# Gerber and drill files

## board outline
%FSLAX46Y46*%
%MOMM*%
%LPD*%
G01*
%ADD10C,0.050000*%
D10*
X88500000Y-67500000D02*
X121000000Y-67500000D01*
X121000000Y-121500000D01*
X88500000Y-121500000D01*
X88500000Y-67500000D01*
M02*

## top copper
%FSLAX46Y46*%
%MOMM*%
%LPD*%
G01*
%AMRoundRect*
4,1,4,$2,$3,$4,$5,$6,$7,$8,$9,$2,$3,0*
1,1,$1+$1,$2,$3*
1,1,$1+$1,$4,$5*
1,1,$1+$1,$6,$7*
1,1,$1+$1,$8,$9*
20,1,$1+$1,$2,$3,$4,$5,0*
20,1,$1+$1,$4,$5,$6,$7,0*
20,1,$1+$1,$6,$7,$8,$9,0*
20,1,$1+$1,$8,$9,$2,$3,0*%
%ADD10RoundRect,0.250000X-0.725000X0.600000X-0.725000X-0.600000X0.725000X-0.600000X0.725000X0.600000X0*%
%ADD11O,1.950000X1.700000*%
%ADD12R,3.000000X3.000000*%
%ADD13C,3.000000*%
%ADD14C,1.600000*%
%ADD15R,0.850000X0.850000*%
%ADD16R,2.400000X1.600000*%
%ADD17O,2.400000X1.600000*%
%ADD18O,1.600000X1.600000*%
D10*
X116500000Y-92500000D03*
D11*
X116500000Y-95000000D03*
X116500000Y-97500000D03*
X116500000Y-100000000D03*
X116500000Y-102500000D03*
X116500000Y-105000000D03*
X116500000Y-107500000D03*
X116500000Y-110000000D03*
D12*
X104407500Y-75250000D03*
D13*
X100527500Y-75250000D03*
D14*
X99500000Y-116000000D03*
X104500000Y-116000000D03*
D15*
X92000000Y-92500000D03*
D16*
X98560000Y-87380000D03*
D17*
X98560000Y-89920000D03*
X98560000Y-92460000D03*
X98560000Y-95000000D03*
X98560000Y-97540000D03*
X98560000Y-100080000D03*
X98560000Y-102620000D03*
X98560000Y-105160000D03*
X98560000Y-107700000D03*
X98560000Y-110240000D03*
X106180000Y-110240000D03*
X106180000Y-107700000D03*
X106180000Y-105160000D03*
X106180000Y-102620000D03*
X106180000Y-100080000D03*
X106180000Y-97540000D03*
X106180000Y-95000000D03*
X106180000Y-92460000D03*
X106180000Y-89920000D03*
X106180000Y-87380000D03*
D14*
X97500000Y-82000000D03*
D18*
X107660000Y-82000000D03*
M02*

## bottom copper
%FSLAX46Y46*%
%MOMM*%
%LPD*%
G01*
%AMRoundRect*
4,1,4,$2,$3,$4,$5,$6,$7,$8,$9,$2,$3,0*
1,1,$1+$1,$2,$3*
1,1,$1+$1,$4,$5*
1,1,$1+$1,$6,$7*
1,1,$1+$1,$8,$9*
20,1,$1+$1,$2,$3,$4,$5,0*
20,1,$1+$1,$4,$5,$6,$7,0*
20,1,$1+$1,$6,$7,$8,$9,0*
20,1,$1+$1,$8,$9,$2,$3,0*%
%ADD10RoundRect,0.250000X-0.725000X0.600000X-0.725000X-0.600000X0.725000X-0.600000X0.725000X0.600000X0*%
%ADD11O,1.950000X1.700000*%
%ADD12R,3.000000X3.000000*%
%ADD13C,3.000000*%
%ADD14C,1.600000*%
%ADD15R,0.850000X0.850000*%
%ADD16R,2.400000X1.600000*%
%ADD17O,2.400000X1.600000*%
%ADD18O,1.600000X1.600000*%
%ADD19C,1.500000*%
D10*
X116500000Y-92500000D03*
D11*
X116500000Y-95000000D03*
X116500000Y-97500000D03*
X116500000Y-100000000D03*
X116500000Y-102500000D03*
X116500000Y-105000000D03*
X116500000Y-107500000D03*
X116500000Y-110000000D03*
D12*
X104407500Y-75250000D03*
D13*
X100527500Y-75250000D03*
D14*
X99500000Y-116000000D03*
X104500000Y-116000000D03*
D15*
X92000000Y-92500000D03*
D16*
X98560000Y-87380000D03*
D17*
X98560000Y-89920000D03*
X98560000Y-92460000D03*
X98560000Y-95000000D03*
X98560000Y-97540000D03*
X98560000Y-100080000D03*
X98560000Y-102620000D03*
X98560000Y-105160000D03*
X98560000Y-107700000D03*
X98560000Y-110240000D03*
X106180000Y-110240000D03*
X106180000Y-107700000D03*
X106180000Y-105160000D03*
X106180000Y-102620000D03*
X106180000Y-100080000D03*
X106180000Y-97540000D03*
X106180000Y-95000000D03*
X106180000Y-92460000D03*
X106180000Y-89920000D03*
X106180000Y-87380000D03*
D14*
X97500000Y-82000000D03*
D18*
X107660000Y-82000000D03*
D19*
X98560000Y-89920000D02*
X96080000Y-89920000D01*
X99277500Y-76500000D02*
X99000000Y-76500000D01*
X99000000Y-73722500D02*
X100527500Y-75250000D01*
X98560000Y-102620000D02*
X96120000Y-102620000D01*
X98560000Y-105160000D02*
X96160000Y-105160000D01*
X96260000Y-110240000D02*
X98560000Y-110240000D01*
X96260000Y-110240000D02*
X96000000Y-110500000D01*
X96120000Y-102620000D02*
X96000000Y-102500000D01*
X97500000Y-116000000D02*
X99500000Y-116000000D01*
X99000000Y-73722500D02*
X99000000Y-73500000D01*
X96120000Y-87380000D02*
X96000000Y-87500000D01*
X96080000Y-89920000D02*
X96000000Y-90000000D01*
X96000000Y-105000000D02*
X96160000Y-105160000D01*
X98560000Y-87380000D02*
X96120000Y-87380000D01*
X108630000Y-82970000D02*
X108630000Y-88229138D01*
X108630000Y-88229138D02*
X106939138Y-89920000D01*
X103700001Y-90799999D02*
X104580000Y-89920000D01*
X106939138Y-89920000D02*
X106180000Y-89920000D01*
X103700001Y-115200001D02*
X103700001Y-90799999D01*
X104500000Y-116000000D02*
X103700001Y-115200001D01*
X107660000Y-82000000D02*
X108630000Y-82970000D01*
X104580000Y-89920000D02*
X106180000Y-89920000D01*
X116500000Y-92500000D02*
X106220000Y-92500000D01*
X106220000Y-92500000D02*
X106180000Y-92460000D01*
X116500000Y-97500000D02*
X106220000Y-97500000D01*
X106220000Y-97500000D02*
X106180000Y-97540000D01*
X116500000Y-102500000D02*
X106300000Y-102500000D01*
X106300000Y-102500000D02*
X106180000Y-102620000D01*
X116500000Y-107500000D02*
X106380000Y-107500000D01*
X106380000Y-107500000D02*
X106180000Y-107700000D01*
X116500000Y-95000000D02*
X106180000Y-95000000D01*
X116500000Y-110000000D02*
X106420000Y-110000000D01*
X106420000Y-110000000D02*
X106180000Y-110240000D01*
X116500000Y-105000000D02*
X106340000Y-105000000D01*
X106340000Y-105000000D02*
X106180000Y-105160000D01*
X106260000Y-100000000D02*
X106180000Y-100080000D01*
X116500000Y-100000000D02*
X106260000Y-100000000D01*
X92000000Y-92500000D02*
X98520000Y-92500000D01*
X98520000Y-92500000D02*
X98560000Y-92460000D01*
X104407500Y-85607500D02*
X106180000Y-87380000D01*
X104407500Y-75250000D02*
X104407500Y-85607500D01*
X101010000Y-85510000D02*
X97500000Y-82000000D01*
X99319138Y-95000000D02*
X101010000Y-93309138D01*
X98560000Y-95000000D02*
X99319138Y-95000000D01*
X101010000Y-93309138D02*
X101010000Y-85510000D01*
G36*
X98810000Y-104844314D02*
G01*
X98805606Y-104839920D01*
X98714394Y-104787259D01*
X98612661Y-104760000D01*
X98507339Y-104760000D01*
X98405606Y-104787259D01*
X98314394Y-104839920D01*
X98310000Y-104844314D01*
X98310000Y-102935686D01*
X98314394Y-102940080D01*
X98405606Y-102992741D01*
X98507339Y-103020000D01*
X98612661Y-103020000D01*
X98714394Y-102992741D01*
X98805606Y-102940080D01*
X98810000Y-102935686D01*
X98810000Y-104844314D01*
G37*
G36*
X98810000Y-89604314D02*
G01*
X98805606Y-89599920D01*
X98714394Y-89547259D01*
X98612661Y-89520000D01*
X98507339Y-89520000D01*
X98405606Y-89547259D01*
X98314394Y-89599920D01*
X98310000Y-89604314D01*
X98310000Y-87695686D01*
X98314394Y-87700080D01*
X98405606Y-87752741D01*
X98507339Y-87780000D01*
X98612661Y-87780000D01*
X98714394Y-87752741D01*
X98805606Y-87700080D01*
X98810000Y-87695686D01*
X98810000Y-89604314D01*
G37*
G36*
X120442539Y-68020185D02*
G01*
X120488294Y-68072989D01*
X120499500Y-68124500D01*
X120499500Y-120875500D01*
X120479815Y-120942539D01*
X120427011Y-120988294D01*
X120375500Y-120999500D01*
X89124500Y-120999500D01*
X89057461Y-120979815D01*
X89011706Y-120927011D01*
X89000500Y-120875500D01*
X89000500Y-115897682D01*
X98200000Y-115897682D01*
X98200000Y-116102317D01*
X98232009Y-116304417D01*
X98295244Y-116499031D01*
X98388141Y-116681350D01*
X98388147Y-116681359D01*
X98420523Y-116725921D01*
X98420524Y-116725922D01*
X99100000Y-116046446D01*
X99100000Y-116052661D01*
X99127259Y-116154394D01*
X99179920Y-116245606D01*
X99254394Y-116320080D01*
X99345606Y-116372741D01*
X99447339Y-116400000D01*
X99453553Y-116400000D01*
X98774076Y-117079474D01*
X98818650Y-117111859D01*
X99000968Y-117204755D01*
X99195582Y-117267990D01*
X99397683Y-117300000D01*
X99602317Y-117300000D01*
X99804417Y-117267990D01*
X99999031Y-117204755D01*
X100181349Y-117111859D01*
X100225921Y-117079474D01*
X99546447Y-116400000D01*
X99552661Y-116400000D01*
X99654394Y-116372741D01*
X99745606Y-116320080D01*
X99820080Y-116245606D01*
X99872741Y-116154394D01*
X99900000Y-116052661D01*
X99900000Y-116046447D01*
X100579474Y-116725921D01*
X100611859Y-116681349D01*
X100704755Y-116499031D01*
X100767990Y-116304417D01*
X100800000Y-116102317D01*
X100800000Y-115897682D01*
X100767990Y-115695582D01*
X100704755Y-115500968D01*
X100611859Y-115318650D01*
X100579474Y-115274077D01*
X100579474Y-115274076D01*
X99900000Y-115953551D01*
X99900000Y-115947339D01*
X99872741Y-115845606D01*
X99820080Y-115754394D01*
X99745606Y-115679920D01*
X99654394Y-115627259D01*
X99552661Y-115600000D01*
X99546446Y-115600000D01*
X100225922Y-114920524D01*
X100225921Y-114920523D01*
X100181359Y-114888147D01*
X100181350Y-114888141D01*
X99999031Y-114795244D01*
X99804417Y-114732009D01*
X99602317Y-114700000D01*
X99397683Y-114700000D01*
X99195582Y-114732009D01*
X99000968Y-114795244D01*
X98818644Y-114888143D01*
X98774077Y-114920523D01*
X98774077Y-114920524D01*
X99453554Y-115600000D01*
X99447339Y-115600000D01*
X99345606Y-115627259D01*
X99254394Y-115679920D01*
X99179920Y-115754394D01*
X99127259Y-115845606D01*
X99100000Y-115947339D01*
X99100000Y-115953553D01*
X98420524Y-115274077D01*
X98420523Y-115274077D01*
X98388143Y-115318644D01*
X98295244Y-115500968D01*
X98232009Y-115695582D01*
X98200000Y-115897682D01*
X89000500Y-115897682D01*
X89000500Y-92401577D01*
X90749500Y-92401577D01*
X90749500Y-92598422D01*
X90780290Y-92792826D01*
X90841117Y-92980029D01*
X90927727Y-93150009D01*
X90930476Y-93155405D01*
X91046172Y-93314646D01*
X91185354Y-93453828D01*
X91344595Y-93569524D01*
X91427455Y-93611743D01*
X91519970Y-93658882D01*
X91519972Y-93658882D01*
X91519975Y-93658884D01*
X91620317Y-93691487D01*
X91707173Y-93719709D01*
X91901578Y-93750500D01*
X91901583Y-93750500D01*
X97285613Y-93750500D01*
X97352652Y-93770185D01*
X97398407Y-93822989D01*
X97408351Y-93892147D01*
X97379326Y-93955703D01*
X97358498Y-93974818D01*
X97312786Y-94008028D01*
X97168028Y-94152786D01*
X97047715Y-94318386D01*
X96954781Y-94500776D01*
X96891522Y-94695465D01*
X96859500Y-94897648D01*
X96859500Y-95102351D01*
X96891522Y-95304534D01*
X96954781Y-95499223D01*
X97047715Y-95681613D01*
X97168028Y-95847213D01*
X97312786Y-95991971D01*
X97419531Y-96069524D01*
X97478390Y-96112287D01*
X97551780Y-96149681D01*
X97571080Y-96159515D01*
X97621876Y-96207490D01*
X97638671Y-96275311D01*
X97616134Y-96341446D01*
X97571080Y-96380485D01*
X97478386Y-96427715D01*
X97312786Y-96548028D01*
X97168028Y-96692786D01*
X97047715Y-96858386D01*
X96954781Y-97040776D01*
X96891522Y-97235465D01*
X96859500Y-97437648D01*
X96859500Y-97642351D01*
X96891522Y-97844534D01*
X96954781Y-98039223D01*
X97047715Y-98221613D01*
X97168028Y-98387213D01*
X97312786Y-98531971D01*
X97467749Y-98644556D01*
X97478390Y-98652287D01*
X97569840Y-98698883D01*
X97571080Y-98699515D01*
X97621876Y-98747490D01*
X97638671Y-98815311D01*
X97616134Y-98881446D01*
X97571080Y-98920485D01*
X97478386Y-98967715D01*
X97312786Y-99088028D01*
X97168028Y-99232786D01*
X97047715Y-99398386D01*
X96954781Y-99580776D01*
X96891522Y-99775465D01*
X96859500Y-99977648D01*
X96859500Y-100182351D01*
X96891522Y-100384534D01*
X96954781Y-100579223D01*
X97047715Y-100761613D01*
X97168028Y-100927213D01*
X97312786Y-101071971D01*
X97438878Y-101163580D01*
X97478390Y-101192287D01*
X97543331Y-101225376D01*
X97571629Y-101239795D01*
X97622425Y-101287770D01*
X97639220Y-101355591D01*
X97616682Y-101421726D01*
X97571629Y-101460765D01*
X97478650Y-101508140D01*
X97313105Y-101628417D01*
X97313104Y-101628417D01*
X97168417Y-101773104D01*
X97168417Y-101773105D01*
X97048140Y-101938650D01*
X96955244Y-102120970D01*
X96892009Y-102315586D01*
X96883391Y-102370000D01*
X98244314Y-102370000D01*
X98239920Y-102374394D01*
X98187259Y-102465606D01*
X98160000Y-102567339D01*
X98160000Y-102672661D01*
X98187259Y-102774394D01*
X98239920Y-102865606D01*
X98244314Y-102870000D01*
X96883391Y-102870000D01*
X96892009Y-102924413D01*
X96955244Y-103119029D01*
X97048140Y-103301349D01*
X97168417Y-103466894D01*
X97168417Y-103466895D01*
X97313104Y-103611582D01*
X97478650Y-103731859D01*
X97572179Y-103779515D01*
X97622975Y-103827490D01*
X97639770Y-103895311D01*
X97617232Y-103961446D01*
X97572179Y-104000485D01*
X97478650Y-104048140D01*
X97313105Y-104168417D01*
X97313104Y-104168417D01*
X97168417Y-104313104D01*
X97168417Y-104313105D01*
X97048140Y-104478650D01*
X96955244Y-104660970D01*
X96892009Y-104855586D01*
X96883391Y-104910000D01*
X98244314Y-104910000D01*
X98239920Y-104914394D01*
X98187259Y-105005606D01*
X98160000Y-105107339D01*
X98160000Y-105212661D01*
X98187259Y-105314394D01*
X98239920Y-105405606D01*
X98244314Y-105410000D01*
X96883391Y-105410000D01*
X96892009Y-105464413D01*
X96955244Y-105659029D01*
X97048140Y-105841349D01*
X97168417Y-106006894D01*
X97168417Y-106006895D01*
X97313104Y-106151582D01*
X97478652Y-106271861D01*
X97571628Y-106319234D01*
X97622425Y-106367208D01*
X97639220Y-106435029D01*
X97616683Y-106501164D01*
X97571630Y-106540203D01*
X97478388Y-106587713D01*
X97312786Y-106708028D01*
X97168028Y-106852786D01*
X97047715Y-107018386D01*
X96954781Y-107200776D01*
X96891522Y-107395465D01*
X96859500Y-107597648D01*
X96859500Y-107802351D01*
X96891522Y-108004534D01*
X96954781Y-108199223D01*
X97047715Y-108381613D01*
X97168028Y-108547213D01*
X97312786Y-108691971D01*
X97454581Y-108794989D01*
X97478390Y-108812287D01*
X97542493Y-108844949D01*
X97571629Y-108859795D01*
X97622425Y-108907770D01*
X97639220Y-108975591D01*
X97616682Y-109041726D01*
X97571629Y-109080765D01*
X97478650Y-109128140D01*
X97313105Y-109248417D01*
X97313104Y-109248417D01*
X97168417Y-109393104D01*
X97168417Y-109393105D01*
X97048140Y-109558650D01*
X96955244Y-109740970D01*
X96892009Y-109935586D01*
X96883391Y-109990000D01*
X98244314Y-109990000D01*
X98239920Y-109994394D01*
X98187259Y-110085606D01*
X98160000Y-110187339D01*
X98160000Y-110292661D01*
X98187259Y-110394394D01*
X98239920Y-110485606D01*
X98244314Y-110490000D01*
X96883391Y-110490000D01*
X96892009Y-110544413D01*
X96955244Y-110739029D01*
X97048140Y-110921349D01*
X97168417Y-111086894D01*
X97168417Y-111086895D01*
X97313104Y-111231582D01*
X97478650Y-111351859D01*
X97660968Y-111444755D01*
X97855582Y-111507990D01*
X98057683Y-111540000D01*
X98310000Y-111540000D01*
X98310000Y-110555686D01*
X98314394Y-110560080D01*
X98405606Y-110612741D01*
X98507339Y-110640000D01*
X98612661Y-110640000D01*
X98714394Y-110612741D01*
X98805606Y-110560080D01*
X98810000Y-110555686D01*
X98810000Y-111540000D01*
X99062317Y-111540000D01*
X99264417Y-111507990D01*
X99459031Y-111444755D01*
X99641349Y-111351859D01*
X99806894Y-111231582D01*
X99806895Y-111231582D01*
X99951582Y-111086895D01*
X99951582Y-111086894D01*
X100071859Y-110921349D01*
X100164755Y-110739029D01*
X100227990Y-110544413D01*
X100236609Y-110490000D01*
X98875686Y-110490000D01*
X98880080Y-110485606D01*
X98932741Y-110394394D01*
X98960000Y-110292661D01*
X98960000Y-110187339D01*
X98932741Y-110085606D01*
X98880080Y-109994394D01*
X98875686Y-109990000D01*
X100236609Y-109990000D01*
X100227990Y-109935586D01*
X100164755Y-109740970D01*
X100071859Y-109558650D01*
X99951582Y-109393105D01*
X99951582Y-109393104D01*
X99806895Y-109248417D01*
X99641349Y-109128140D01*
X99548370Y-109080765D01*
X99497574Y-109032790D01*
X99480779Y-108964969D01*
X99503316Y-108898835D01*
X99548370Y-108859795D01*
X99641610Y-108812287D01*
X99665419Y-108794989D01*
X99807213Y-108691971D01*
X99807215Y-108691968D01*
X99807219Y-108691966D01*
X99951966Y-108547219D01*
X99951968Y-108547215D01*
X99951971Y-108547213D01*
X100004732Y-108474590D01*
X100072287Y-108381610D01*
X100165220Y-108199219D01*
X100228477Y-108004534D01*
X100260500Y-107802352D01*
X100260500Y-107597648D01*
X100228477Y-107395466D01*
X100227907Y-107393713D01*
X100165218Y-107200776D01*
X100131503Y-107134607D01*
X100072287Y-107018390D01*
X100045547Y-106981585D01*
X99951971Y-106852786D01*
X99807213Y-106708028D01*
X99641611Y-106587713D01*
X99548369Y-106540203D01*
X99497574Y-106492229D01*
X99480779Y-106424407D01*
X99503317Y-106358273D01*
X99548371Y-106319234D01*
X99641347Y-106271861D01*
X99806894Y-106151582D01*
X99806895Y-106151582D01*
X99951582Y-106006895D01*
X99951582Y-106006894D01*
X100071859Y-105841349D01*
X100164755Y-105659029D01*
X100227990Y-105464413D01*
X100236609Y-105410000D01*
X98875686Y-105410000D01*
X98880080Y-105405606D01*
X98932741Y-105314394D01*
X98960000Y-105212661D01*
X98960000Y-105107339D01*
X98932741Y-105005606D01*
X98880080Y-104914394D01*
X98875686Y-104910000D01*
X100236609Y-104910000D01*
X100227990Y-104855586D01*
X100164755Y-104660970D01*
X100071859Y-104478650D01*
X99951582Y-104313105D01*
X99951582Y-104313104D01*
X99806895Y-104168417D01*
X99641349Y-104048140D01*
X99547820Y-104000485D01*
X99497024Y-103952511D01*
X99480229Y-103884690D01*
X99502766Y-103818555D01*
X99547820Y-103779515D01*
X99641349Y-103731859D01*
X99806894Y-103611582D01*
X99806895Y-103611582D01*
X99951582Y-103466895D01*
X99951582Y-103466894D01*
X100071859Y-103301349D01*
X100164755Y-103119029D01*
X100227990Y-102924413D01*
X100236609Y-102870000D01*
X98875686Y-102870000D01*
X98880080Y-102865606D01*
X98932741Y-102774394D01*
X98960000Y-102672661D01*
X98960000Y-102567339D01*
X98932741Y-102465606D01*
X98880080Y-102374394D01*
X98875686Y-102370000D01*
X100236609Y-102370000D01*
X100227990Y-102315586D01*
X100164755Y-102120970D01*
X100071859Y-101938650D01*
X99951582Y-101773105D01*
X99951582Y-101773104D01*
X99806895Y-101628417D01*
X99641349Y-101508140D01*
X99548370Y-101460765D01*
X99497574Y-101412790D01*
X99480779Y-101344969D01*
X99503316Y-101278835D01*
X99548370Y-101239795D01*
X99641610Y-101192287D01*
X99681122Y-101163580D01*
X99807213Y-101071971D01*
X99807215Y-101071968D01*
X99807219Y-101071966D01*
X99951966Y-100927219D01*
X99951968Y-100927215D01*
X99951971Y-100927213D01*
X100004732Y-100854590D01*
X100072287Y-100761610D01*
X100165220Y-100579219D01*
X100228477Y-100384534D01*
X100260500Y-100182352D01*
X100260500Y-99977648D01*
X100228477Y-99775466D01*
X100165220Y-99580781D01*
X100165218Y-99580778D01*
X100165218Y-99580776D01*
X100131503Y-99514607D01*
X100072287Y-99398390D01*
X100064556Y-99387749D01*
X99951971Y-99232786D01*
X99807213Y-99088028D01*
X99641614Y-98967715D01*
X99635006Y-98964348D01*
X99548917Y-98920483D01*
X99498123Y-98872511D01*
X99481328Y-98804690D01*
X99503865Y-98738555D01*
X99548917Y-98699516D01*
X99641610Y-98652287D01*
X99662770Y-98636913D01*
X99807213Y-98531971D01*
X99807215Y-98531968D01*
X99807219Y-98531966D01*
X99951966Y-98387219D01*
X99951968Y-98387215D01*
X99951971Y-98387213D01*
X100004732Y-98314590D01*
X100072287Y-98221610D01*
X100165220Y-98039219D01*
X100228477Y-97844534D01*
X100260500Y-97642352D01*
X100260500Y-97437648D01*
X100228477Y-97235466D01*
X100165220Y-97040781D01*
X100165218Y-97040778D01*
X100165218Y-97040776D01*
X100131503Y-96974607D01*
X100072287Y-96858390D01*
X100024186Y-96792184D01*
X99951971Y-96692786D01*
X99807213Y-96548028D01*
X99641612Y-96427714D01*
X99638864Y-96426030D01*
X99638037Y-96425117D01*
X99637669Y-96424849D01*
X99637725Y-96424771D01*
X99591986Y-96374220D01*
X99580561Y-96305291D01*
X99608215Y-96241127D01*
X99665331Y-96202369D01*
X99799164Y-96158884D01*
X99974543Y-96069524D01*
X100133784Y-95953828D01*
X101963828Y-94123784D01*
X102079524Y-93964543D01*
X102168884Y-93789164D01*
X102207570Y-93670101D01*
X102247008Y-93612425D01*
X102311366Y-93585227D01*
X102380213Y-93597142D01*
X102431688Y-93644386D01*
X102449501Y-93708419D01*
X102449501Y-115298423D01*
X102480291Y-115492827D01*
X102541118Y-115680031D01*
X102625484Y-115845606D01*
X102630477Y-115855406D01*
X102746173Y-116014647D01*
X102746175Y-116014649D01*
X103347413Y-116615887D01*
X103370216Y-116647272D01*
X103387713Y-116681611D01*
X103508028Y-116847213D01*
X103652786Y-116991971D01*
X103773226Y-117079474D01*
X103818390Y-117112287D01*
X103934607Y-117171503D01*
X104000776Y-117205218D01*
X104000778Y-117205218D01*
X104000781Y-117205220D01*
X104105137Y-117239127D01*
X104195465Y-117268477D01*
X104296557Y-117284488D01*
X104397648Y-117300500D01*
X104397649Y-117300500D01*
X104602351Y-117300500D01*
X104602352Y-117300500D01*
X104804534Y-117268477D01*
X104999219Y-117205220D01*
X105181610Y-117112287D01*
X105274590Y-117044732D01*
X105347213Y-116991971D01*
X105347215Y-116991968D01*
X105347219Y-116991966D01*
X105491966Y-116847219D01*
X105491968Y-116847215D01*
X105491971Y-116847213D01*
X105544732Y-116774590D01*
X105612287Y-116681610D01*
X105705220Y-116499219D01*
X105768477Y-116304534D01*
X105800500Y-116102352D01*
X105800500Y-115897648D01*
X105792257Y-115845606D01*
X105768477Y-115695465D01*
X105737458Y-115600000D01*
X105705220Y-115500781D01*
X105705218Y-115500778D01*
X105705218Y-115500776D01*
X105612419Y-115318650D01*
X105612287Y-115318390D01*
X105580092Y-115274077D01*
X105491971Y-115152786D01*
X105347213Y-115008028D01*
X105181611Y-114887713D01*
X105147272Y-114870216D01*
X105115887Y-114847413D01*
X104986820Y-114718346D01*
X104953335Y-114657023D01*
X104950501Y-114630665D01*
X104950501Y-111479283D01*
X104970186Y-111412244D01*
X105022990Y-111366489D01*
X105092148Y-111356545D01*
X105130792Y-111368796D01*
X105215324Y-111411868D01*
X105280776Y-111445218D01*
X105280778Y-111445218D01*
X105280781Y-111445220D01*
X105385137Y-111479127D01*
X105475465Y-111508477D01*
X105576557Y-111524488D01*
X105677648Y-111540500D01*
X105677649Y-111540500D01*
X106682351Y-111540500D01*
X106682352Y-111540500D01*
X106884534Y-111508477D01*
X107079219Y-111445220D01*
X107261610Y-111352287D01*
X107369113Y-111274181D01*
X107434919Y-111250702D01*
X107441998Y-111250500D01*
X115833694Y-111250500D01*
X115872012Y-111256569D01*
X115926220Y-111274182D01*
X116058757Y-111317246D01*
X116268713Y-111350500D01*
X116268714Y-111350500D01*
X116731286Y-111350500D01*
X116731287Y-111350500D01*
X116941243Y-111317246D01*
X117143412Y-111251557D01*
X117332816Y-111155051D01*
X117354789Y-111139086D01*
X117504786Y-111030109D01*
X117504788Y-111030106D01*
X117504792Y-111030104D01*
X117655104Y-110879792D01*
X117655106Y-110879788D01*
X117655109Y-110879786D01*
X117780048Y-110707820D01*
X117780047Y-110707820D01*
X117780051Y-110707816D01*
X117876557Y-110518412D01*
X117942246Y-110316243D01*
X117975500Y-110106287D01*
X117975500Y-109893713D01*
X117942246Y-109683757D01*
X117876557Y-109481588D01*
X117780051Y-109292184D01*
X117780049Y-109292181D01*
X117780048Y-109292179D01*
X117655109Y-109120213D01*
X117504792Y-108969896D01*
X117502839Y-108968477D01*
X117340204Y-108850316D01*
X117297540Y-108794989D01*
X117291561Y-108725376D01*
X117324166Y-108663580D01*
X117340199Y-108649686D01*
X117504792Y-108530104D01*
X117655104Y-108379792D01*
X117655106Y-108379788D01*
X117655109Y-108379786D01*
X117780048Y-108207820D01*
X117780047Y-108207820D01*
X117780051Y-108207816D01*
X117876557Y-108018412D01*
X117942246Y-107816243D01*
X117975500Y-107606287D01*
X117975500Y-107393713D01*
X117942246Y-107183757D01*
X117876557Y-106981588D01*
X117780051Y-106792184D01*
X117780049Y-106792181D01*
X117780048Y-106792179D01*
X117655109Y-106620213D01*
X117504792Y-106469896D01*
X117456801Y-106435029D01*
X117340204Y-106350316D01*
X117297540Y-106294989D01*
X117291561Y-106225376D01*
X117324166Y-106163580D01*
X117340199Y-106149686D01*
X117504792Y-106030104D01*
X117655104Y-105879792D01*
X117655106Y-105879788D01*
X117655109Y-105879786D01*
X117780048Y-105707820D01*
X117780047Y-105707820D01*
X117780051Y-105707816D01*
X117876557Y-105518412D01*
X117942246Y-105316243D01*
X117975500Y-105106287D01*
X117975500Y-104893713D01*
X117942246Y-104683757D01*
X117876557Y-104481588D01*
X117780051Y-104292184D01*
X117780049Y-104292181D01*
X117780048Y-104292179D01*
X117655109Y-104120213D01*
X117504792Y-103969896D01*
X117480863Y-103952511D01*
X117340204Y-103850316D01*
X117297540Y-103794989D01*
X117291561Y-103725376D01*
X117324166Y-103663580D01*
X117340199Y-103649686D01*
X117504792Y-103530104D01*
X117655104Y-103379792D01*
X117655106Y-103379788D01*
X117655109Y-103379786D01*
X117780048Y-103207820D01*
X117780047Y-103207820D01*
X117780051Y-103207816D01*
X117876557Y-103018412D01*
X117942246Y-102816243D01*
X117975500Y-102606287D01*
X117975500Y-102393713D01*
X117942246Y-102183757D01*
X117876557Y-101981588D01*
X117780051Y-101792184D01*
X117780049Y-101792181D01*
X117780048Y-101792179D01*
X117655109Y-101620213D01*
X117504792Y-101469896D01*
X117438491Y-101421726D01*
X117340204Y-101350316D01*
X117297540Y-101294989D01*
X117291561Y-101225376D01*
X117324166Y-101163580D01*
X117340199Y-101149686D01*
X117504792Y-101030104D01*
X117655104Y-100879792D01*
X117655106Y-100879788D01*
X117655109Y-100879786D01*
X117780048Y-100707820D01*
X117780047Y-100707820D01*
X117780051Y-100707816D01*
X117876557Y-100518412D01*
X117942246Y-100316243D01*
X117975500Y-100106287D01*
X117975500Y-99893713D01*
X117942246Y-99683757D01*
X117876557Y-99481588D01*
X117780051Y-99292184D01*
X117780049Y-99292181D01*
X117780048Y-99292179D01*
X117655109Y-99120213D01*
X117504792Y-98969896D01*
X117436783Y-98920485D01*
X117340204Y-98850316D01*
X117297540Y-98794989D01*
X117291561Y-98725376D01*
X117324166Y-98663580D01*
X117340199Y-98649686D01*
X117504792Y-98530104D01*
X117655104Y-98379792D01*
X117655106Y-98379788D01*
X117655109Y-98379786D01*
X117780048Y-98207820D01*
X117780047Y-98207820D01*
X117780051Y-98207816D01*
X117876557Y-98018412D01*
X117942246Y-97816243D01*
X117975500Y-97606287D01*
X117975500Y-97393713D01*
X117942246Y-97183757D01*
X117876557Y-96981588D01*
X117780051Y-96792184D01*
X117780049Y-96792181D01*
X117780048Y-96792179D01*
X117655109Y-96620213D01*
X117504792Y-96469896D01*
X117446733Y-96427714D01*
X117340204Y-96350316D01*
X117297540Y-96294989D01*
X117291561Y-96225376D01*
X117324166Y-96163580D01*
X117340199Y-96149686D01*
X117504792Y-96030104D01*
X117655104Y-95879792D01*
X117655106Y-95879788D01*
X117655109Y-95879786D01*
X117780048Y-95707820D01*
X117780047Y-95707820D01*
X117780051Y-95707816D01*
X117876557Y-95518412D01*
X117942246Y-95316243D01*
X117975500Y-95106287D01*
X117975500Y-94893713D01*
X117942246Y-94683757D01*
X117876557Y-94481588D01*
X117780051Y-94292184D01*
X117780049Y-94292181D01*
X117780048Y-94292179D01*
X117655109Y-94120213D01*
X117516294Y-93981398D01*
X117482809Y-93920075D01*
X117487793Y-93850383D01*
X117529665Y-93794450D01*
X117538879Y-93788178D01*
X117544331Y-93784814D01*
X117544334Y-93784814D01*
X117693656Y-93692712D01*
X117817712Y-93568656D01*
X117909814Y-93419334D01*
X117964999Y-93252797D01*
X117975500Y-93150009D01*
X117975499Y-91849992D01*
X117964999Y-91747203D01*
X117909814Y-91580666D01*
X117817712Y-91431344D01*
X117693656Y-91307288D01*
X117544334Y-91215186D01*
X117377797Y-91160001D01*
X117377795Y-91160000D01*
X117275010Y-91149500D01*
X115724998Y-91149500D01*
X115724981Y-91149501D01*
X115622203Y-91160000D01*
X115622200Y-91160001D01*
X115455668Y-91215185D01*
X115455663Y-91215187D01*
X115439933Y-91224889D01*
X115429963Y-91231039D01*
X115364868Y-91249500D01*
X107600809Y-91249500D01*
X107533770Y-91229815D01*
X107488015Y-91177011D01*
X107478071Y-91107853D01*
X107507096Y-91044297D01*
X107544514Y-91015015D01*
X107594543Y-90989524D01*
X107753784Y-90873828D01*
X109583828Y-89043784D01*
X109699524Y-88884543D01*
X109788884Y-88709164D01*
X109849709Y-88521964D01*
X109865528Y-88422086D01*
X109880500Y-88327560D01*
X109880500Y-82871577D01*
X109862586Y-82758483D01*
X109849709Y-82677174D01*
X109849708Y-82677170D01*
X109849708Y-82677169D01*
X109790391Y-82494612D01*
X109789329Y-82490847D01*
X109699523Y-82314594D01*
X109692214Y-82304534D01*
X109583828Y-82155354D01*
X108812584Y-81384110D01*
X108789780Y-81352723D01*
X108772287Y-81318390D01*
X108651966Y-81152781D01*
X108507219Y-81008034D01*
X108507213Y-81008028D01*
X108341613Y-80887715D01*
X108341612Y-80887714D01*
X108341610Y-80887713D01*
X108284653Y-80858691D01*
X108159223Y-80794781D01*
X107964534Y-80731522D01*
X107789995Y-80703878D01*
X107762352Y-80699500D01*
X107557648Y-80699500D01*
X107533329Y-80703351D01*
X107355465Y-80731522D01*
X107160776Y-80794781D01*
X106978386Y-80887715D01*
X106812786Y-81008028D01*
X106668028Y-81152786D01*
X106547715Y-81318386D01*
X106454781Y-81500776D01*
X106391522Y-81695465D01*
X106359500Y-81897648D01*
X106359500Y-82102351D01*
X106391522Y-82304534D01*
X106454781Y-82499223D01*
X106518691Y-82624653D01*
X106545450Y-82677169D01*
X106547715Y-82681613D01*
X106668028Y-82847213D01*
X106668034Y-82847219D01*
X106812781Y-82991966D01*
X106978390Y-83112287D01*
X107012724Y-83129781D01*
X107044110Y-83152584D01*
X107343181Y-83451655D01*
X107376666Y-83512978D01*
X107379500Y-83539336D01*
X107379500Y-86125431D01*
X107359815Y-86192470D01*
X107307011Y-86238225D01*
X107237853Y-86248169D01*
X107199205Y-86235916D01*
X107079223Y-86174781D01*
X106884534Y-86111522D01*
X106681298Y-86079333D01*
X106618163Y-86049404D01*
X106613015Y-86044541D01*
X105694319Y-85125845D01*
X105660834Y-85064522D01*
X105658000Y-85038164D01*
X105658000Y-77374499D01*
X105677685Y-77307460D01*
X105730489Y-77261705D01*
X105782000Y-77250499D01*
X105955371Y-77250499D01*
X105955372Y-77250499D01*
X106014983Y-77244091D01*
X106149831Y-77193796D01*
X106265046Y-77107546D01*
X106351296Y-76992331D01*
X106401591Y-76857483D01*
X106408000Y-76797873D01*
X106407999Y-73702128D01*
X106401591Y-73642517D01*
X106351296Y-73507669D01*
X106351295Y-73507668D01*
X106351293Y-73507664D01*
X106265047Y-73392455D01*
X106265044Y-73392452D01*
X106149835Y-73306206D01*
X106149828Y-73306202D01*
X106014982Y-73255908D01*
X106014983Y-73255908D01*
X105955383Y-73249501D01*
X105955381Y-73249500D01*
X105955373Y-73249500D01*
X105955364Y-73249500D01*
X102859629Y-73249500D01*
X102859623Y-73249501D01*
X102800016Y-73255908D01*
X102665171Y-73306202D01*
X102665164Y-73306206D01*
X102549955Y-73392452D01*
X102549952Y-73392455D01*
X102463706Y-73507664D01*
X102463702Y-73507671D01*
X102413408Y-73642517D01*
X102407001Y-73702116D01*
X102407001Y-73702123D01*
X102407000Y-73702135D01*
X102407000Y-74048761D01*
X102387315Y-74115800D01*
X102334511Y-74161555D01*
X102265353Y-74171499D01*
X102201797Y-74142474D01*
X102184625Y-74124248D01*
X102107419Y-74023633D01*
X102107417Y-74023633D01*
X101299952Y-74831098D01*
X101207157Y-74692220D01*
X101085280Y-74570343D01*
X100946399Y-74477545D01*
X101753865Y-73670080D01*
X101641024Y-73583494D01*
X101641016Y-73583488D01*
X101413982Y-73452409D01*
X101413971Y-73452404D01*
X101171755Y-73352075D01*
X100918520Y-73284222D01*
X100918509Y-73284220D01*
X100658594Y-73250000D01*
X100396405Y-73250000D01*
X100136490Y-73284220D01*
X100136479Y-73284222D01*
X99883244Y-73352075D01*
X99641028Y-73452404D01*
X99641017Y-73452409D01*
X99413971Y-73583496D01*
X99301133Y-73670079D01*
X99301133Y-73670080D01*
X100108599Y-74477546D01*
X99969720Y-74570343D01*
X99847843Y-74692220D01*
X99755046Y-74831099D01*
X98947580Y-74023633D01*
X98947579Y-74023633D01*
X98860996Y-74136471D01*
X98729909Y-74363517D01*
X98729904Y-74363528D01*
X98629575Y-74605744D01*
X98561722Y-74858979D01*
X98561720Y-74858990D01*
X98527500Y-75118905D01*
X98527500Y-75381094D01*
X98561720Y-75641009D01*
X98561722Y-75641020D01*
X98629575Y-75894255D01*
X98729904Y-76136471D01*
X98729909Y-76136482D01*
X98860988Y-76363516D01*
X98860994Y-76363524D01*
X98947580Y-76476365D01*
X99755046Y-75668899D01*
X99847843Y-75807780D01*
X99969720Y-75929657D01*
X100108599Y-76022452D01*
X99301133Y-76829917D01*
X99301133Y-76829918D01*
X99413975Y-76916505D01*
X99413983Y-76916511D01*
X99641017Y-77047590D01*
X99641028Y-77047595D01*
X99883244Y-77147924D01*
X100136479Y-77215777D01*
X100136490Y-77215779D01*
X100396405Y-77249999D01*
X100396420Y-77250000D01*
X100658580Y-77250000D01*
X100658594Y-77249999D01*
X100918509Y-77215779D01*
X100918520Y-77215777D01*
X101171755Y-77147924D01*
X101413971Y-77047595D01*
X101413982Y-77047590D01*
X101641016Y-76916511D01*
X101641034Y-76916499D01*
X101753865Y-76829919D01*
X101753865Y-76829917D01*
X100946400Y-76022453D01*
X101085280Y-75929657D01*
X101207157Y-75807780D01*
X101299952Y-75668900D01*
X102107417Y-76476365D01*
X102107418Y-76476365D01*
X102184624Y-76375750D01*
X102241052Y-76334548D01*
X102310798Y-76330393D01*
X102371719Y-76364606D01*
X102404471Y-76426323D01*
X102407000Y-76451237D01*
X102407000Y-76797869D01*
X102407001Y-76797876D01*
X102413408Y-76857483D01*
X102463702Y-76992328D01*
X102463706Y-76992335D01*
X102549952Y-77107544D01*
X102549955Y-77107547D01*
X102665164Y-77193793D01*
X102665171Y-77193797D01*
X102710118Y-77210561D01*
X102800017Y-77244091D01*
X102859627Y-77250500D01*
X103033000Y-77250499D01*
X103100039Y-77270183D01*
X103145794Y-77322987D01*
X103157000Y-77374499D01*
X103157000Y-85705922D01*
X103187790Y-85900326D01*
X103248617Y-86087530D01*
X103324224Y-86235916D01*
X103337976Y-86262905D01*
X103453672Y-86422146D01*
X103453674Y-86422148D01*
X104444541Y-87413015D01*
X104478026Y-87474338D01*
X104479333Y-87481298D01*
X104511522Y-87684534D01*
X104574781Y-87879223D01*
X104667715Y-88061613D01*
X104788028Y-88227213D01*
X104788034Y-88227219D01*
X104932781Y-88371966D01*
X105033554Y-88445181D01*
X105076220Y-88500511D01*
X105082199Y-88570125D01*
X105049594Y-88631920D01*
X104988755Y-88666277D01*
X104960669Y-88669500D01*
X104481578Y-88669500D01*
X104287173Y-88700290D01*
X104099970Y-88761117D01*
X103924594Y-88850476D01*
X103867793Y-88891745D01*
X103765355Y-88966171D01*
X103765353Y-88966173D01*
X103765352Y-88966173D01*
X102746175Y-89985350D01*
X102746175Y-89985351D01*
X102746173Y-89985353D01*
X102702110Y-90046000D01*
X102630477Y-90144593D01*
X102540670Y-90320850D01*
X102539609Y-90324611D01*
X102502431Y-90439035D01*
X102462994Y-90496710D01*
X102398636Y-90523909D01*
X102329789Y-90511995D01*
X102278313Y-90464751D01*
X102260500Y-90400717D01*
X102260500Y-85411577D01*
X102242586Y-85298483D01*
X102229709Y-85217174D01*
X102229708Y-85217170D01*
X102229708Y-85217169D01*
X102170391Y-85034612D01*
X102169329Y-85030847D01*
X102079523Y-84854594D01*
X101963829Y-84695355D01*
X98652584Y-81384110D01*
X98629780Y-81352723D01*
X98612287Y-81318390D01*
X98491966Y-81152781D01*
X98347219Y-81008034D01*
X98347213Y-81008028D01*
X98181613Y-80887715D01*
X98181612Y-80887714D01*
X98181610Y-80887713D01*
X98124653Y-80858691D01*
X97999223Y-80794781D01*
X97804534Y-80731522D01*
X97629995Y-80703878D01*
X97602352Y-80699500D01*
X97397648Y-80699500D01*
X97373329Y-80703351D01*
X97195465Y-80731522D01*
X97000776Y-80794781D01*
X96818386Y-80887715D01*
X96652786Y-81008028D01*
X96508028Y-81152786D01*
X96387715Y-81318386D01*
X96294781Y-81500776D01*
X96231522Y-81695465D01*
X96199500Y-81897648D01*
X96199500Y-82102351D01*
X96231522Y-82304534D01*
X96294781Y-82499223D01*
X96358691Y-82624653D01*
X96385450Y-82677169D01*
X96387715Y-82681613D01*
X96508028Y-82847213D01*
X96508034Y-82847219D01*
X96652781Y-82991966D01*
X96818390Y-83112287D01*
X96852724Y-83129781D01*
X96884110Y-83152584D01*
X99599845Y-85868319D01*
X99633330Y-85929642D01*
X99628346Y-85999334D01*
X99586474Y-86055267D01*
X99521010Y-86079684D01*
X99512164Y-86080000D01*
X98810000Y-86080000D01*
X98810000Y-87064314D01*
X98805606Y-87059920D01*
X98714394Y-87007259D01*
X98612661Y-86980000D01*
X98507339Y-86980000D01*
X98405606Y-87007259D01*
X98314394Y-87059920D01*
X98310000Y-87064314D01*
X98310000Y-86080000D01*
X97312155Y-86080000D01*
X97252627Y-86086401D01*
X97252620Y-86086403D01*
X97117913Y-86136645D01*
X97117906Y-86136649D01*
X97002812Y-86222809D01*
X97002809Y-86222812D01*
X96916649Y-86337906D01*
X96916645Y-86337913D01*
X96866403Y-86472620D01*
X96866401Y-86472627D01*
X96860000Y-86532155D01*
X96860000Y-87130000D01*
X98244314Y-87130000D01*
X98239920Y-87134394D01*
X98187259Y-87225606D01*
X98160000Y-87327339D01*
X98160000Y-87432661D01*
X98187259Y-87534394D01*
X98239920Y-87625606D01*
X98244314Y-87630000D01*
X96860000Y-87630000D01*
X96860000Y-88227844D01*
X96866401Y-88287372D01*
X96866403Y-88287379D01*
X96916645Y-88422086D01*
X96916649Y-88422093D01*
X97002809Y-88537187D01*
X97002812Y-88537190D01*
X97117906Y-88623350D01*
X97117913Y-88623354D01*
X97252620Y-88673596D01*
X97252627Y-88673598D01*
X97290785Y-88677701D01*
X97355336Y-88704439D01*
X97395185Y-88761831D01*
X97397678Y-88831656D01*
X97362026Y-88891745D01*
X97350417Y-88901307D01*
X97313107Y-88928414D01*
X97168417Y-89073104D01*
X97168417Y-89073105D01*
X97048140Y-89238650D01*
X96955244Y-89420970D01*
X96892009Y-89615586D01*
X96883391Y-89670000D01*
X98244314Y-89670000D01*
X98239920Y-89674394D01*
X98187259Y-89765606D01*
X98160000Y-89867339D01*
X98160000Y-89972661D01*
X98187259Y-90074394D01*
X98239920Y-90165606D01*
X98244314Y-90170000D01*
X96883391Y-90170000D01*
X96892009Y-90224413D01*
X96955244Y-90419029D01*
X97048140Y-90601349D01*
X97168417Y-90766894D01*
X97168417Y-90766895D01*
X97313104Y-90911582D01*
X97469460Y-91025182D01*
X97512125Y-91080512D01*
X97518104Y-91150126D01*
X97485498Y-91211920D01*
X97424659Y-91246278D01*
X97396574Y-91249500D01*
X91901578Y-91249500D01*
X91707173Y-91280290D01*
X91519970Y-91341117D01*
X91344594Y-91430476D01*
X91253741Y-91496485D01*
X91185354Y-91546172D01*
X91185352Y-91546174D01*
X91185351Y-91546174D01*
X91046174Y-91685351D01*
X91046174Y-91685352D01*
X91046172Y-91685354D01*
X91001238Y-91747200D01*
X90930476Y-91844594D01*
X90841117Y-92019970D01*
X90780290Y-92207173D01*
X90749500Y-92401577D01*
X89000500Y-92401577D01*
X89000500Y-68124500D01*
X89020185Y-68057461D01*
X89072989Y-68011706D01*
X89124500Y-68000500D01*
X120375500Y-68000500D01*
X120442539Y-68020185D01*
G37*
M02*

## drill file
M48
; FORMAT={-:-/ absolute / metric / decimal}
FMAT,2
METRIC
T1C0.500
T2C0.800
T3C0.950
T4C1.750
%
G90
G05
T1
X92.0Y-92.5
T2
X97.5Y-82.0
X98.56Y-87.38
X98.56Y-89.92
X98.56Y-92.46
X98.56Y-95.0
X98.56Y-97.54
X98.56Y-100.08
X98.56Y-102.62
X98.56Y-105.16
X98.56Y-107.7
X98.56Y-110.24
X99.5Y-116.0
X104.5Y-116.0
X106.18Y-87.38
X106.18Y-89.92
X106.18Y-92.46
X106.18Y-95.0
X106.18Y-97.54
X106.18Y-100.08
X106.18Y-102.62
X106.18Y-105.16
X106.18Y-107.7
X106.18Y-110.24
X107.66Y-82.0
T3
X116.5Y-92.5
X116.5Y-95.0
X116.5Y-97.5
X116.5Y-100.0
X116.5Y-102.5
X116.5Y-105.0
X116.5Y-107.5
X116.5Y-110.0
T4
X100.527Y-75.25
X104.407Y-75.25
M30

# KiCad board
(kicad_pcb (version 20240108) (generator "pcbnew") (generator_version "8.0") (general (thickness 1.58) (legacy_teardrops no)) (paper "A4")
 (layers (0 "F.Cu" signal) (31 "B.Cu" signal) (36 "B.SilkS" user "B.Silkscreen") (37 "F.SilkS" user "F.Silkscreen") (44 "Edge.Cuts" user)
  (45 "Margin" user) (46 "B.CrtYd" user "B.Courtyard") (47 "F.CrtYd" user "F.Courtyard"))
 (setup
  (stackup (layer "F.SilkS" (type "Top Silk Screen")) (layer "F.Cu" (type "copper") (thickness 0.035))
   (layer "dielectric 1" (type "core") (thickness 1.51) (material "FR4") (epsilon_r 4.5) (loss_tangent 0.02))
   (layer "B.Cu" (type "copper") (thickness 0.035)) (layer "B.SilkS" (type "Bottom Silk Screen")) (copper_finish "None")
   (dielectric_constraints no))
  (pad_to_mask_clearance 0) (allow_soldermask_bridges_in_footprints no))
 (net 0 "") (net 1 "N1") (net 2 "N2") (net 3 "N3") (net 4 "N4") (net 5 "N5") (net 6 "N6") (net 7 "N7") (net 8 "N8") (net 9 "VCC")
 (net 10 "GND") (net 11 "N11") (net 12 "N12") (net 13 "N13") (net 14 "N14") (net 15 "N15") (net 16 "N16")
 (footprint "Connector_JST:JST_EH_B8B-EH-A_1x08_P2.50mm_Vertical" (layer "F.Cu") (at 116.5 92.5 -90)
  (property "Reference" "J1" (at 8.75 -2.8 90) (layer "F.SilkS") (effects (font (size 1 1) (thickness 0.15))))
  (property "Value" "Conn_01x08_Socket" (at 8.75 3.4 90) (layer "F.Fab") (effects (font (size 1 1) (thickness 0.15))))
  (pad "1" thru_hole roundrect (at 0 0 270) (size 1.7 1.95) (drill 0.95) (layers "*.Cu" "*.Mask") (remove_unused_layers no)
   (roundrect_rratio 0.147059) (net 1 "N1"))
  (pad "2" thru_hole oval (at 2.5 0 270) (size 1.7 1.95) (drill 0.95) (layers "*.Cu" "*.Mask") (remove_unused_layers no) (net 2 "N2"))
  (pad "3" thru_hole oval (at 5 0 270) (size 1.7 1.95) (drill 0.95) (layers "*.Cu" "*.Mask") (remove_unused_layers no) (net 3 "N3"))
  (pad "4" thru_hole oval (at 7.5 0 270) (size 1.7 1.95) (drill 0.95) (layers "*.Cu" "*.Mask") (remove_unused_layers no) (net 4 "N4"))
  (pad "5" thru_hole oval (at 10 0 270) (size 1.7 1.95) (drill 0.95) (layers "*.Cu" "*.Mask") (remove_unused_layers no) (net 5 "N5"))
  (pad "6" thru_hole oval (at 12.5 0 270) (size 1.7 1.95) (drill 0.95) (layers "*.Cu" "*.Mask") (remove_unused_layers no) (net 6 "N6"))
  (pad "7" thru_hole oval (at 15 0 270) (size 1.7 1.95) (drill 0.95) (layers "*.Cu" "*.Mask") (remove_unused_layers no) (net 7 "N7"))
  (pad "8" thru_hole oval (at 17.5 0 270) (size 1.7 1.95) (drill 0.95) (layers "*.Cu" "*.Mask") (remove_unused_layers no) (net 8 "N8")))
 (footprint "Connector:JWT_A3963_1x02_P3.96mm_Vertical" (layer "F.Cu") (at 104.4075 75.25 180)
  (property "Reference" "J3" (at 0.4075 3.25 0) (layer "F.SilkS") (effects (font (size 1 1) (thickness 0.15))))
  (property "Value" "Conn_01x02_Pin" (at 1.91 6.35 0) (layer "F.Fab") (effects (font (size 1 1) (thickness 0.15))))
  (pad "1" thru_hole rect (at 0 0 180) (size 3 3) (drill 1.75) (layers "*.Cu" "*.Mask") (remove_unused_layers no) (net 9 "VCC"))
  (pad "2" thru_hole circle (at 3.88 0 180) (size 3 3) (drill 1.75) (layers "*.Cu" "*.Mask") (remove_unused_layers no) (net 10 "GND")))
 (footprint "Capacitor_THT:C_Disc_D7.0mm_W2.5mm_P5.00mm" (layer "F.Cu") (at 99.5 116)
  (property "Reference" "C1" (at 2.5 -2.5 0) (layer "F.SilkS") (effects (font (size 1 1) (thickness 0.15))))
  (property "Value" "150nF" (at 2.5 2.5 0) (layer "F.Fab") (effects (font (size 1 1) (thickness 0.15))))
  (pad "1" thru_hole circle (at 0 0) (size 1.6 1.6) (drill 0.8) (layers "*.Cu" "*.Mask") (remove_unused_layers no) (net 10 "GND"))
  (pad "2" thru_hole circle (at 5 0) (size 1.6 1.6) (drill 0.8) (layers "*.Cu" "*.Mask") (remove_unused_layers no) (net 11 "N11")))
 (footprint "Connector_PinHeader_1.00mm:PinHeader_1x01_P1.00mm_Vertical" (layer "F.Cu") (at 92 92.5)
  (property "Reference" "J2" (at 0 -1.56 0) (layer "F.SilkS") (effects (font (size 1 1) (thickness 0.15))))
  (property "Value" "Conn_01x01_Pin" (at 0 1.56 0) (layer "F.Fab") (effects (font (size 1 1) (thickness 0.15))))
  (pad "1" thru_hole rect (at 0 0) (size 0.85 0.85) (drill 0.5) (layers "*.Cu" "*.Mask") (remove_unused_layers no) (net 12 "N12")))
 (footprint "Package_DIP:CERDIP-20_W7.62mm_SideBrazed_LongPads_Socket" (layer "F.Cu") (at 98.56 87.38)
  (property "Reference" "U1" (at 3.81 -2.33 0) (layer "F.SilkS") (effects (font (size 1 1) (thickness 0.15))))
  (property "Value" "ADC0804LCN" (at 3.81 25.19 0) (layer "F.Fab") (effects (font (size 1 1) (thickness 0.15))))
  (pad "1" thru_hole rect (at 0 0) (size 2.4 1.6) (drill 0.8) (layers "*.Cu" "*.Mask") (remove_unused_layers no) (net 10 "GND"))
  (pad "2" thru_hole oval (at 0 2.54) (size 2.4 1.6) (drill 0.8) (layers "*.Cu" "*.Mask") (remove_unused_layers no) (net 10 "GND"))
  (pad "3" thru_hole oval (at 0 5.08) (size 2.4 1.6) (drill 0.8) (layers "*.Cu" "*.Mask") (remove_unused_layers no) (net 12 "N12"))
  (pad "4" thru_hole oval (at 0 7.62) (size 2.4 1.6) (drill 0.8) (layers "*.Cu" "*.Mask") (remove_unused_layers no) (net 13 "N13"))
  (pad "5" thru_hole oval (at 0 10.16) (size 2.4 1.6) (drill 0.8) (layers "*.Cu" "*.Mask") (remove_unused_layers no) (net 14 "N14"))
  (pad "6" thru_hole oval (at 0 12.7) (size 2.4 1.6) (drill 0.8) (layers "*.Cu" "*.Mask") (remove_unused_layers no) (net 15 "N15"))
  (pad "7" thru_hole oval (at 0 15.24) (size 2.4 1.6) (drill 0.8) (layers "*.Cu" "*.Mask") (remove_unused_layers no) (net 10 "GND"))
  (pad "8" thru_hole oval (at 0 17.78) (size 2.4 1.6) (drill 0.8) (layers "*.Cu" "*.Mask") (remove_unused_layers no) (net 10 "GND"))
  (pad "9" thru_hole oval (at 0 20.32) (size 2.4 1.6) (drill 0.8) (layers "*.Cu" "*.Mask") (remove_unused_layers no) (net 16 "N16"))
  (pad "10" thru_hole oval (at 0 22.86) (size 2.4 1.6) (drill 0.8) (layers "*.Cu" "*.Mask") (remove_unused_layers no) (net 10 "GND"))
  (pad "11" thru_hole oval (at 7.62 22.86) (size 2.4 1.6) (drill 0.8) (layers "*.Cu" "*.Mask") (remove_unused_layers no) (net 8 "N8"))
  (pad "12" thru_hole oval (at 7.62 20.32) (size 2.4 1.6) (drill 0.8) (layers "*.Cu" "*.Mask") (remove_unused_layers no) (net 7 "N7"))
  (pad "13" thru_hole oval (at 7.62 17.78) (size 2.4 1.6) (drill 0.8) (layers "*.Cu" "*.Mask") (remove_unused_layers no) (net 6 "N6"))
  (pad "14" thru_hole oval (at 7.62 15.24) (size 2.4 1.6) (drill 0.8) (layers "*.Cu" "*.Mask") (remove_unused_layers no) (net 5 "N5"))
  (pad "15" thru_hole oval (at 7.62 12.7) (size 2.4 1.6) (drill 0.8) (layers "*.Cu" "*.Mask") (remove_unused_layers no) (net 4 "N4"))
  (pad "16" thru_hole oval (at 7.62 10.16) (size 2.4 1.6) (drill 0.8) (layers "*.Cu" "*.Mask") (remove_unused_layers no) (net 3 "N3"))
  (pad "17" thru_hole oval (at 7.62 7.62) (size 2.4 1.6) (drill 0.8) (layers "*.Cu" "*.Mask") (remove_unused_layers no) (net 2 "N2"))
  (pad "18" thru_hole oval (at 7.62 5.08) (size 2.4 1.6) (drill 0.8) (layers "*.Cu" "*.Mask") (remove_unused_layers no) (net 1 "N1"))
  (pad "19" thru_hole oval (at 7.62 2.54) (size 2.4 1.6) (drill 0.8) (layers "*.Cu" "*.Mask") (remove_unused_layers no) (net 11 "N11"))
  (pad "20" thru_hole oval (at 7.62 0) (size 2.4 1.6) (drill 0.8) (layers "*.Cu" "*.Mask") (remove_unused_layers no) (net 9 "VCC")))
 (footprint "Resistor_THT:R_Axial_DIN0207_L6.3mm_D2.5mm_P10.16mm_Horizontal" (layer "F.Cu") (at 97.5 82)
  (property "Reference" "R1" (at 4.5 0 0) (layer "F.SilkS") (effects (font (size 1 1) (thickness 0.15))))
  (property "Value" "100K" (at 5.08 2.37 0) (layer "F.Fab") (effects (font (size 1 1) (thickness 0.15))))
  (pad "1" thru_hole circle (at 0 0) (size 1.6 1.6) (drill 0.8) (layers "*.Cu" "*.Mask") (remove_unused_layers no) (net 13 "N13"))
  (pad "2" thru_hole oval (at 10.16 0) (size 1.6 1.6) (drill 0.8) (layers "*.Cu" "*.Mask") (remove_unused_layers no) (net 11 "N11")))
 (gr_rect (start 88.5 67.5) (end 121 121.5) (stroke (width 0.05) (type default)) (fill none) (layer "Edge.Cuts"))
 (segment (start 98.56 89.92) (end 96.08 89.92) (width 1.5) (layer "B.Cu") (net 10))
 (segment (start 99.2775 76.5) (end 99 76.5) (width 1.5) (layer "B.Cu") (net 10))
 (segment (start 99 73.7225) (end 100.5275 75.25) (width 1.5) (layer "B.Cu") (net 10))
 (segment (start 98.56 102.62) (end 96.12 102.62) (width 1.5) (layer "B.Cu") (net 10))
 (segment (start 98.56 105.16) (end 96.16 105.16) (width 1.5) (layer "B.Cu") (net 10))
 (segment (start 96.26 110.24) (end 98.56 110.24) (width 1.5) (layer "B.Cu") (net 10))
 (segment (start 96.26 110.24) (end 96 110.5) (width 1.5) (layer "B.Cu") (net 10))
 (segment (start 96.12 102.62) (end 96 102.5) (width 1.5) (layer "B.Cu") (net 10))
 (segment (start 97.5 116) (end 99.5 116) (width 1.5) (layer "B.Cu") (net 10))
 (segment (start 99 73.7225) (end 99 73.5) (width 1.5) (layer "B.Cu") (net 10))
 (segment (start 96.12 87.38) (end 96 87.5) (width 1.5) (layer "B.Cu") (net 10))
 (segment (start 96.08 89.92) (end 96 90) (width 1.5) (layer "B.Cu") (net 10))
 (segment (start 96 105) (end 96.16 105.16) (width 1.5) (layer "B.Cu") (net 10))
 (segment (start 98.56 87.38) (end 96.12 87.38) (width 1.5) (layer "B.Cu") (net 10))
 (segment (start 108.63 82.97) (end 108.63 88.229138) (width 1.5) (layer "B.Cu") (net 11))
 (segment (start 108.63 88.229138) (end 106.939138 89.92) (width 1.5) (layer "B.Cu") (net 11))
 (segment (start 103.700001 90.799999) (end 104.58 89.92) (width 1.5) (layer "B.Cu") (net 11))
 (segment (start 106.939138 89.92) (end 106.18 89.92) (width 1.5) (layer "B.Cu") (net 11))
 (segment (start 103.700001 115.200001) (end 103.700001 90.799999) (width 1.5) (layer "B.Cu") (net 11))
 (segment (start 104.5 116) (end 103.700001 115.200001) (width 1.5) (layer "B.Cu") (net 11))
 (segment (start 107.66 82) (end 108.63 82.97) (width 1.5) (layer "B.Cu") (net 11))
 (segment (start 104.58 89.92) (end 106.18 89.92) (width 1.5) (layer "B.Cu") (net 11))
 (segment (start 116.5 92.5) (end 106.22 92.5) (width 1.5) (layer "B.Cu") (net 1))
 (segment (start 106.22 92.5) (end 106.18 92.46) (width 1.5) (layer "B.Cu") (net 1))
 (segment (start 116.5 97.5) (end 106.22 97.5) (width 1.5) (layer "B.Cu") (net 3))
 (segment (start 106.22 97.5) (end 106.18 97.54) (width 1.5) (layer "B.Cu") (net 3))
 (segment (start 116.5 102.5) (end 106.3 102.5) (width 1.5) (layer "B.Cu") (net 5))
 (segment (start 106.3 102.5) (end 106.18 102.62) (width 1.5) (layer "B.Cu") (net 5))
 (segment (start 116.5 107.5) (end 106.38 107.5) (width 1.5) (layer "B.Cu") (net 7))
 (segment (start 106.38 107.5) (end 106.18 107.7) (width 1.5) (layer "B.Cu") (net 7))
 (segment (start 116.5 95) (end 106.18 95) (width 1.5) (layer "B.Cu") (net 2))
 (segment (start 116.5 110) (end 106.42 110) (width 1.5) (layer "B.Cu") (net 8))
 (segment (start 106.42 110) (end 106.18 110.24) (width 1.5) (layer "B.Cu") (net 8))
 (segment (start 116.5 105) (end 106.34 105) (width 1.5) (layer "B.Cu") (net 6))
 (segment (start 106.34 105) (end 106.18 105.16) (width 1.5) (layer "B.Cu") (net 6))
 (segment (start 106.26 100) (end 106.18 100.08) (width 1.5) (layer "B.Cu") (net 4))
 (segment (start 116.5 100) (end 106.26 100) (width 1.5) (layer "B.Cu") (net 4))
 (segment (start 92 92.5) (end 98.52 92.5) (width 1.5) (layer "B.Cu") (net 12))
 (segment (start 98.52 92.5) (end 98.56 92.46) (width 1.5) (layer "B.Cu") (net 12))
 (segment (start 104.4075 85.6075) (end 106.18 87.38) (width 1.5) (layer "B.Cu") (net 9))
 (segment (start 104.4075 75.25) (end 104.4075 85.6075) (width 1.5) (layer "B.Cu") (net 9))
 (segment (start 101.01 85.51) (end 97.5 82) (width 1.5) (layer "B.Cu") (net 13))
 (segment (start 99.319138 95) (end 101.01 93.309138) (width 1.5) (layer "B.Cu") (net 13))
 (segment (start 98.56 95) (end 99.319138 95) (width 1.5) (layer "B.Cu") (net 13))
 (segment (start 101.01 93.309138) (end 101.01 85.51) (width 1.5) (layer "B.Cu") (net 13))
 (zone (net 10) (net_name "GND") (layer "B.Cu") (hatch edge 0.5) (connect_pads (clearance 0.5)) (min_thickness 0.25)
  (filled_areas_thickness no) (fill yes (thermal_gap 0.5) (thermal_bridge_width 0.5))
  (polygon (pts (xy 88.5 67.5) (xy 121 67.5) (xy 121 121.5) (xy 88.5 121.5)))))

